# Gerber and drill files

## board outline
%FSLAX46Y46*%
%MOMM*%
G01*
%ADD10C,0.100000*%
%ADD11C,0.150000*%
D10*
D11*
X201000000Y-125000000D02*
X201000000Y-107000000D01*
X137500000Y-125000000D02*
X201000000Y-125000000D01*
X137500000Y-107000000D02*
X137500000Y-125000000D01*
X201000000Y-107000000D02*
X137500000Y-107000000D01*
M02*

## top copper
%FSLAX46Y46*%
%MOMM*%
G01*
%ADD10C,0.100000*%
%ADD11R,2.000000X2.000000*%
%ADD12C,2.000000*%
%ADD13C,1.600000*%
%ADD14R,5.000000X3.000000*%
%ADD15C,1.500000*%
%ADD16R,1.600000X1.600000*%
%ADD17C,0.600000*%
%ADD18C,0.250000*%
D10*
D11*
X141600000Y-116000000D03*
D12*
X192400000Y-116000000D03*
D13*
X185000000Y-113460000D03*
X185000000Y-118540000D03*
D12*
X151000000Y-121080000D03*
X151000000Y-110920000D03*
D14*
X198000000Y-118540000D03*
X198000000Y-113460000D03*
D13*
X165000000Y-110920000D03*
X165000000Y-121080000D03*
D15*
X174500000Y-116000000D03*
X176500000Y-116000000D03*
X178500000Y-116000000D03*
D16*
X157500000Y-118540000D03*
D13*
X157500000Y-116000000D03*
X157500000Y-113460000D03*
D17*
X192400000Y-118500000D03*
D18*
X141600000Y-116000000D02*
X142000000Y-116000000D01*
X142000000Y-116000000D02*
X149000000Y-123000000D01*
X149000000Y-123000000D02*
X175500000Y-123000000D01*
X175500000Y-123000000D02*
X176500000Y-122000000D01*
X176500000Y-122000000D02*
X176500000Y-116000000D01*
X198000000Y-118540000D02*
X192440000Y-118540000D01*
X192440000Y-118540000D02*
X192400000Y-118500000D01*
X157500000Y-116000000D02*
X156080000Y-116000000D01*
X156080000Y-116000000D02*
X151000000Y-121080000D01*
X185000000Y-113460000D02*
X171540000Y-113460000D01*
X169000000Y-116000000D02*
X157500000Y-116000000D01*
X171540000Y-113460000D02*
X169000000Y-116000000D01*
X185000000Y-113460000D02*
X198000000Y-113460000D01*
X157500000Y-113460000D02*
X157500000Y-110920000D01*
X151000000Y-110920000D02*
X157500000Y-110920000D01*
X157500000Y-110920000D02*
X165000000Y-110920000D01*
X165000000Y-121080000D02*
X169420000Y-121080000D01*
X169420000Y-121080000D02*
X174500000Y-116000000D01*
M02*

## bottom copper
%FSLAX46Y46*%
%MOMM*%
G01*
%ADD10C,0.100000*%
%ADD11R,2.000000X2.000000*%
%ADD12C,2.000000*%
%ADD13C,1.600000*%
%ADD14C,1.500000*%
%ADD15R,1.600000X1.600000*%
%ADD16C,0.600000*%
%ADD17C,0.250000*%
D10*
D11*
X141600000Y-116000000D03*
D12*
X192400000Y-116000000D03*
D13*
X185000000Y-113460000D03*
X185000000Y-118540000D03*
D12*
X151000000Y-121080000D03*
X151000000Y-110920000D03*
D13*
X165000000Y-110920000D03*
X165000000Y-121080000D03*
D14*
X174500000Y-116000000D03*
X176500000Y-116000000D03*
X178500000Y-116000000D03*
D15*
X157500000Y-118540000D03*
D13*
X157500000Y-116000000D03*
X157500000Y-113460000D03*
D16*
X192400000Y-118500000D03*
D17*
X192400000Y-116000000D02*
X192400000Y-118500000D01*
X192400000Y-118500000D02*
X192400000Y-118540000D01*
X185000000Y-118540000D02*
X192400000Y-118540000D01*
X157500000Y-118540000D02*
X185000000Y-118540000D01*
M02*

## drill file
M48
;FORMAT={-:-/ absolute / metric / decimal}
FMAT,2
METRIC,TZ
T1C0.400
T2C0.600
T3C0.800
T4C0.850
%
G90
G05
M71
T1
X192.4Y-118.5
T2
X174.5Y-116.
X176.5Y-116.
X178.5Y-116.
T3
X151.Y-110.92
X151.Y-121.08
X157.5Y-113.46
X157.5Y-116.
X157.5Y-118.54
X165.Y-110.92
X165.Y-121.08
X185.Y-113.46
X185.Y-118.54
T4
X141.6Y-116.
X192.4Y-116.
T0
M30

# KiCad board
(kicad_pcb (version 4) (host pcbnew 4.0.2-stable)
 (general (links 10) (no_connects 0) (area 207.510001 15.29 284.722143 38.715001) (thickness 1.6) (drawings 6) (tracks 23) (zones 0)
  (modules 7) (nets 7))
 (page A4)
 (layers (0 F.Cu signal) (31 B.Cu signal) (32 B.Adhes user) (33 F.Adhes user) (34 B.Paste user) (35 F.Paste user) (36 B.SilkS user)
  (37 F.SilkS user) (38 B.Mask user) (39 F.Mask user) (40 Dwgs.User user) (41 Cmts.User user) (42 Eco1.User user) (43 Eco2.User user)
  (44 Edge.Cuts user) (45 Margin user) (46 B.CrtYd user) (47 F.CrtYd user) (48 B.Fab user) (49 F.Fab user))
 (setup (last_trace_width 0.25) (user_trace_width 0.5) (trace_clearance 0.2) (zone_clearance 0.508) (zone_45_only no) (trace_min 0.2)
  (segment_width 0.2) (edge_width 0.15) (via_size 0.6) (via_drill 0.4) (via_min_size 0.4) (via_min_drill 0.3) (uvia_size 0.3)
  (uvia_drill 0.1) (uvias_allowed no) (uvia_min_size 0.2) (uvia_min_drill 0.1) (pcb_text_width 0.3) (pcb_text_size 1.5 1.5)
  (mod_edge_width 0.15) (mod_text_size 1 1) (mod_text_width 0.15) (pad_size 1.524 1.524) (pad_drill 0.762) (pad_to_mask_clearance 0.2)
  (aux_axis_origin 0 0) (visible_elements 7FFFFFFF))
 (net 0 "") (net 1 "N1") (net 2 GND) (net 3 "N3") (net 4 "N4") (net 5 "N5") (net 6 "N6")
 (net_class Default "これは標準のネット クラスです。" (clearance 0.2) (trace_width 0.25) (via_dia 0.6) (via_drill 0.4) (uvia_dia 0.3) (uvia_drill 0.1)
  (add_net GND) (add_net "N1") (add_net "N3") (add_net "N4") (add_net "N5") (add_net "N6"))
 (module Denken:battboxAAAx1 (layer B.Cu) (at 247.01 29.64)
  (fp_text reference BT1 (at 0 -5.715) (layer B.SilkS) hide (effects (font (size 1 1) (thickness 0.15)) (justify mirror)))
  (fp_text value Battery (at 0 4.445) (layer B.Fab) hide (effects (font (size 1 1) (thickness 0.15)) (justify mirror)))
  (pad 1 thru_hole rect (at -25.4 0) (size 2 2) (drill 0.85) (layers *.Cu *.Mask B.SilkS) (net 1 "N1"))
  (pad 2 thru_hole circle (at 25.4 0) (size 2 2) (drill 0.85) (layers *.Cu *.Mask B.SilkS) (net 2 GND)))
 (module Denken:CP (layer F.Cu) (at 265.01 29.64 270)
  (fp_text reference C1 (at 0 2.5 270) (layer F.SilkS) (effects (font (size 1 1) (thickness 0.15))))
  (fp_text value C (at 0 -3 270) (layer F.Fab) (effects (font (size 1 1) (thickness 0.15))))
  (pad 1 thru_hole circle (at -2.54 0 270) (size 1.6 1.6) (drill 0.8) (layers *.Cu *.Mask F.SilkS) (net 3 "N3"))
  (pad 2 thru_hole circle (at 2.54 0 270) (size 1.6 1.6) (drill 0.8) (layers *.Cu *.Mask F.SilkS) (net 2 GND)))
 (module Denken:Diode (layer F.Cu) (at 231.01 29.64 90)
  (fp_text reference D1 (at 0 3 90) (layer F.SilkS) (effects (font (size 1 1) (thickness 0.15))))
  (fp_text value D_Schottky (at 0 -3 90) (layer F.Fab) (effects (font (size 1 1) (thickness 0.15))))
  (pad 1 thru_hole circle (at -5.08 0 90) (size 2 2) (drill 0.8) (layers *.Cu *.Mask F.SilkS) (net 3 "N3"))
  (pad 2 thru_hole circle (at 5.08 0 90) (size 2 2) (drill 0.8) (layers *.Cu *.Mask F.SilkS) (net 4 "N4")))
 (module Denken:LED (layer F.Cu) (at 278.01 29.64 180)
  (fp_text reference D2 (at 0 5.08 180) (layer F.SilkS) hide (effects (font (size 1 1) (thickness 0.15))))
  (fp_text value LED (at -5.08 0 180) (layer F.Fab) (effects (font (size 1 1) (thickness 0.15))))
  (pad 1 smd rect (at 0 -2.54 180) (size 5 3) (layers F.Cu F.Paste F.Mask) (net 2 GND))
  (pad 2 smd rect (at 0 2.54 180) (size 5 3) (layers F.Cu F.Paste F.Mask) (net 3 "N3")))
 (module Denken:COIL (layer F.Cu) (at 245.01 29.64 270)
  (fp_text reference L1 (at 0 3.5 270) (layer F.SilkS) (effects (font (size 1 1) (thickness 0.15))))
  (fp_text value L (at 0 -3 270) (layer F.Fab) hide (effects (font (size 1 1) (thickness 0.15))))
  (pad 1 thru_hole circle (at -5.08 0 270) (size 1.6 1.6) (drill 0.8) (layers *.Cu *.Mask F.SilkS) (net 4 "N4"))
  (pad 2 thru_hole circle (at 5.08 0 270) (size 1.6 1.6) (drill 0.8) (layers *.Cu *.Mask F.SilkS) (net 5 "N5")))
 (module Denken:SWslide (layer F.Cu) (at 256.51 29.64)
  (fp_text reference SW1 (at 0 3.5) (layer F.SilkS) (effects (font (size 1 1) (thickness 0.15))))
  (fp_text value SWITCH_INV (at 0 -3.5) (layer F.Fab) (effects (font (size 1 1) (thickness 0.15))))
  (pad 1 thru_hole circle (at -2 0) (size 1.5 1.5) (drill 0.6) (layers *.Cu *.Mask F.SilkS) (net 5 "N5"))
  (pad 2 thru_hole circle (at 0 0) (size 1.5 1.5) (drill 0.6) (layers *.Cu *.Mask F.SilkS) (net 1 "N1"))
  (pad 3 thru_hole circle (at 2 0) (size 1.5 1.5) (drill 0.6) (layers *.Cu *.Mask F.SilkS) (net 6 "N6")))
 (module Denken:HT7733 (layer F.Cu) (at 237.51 29.64 90)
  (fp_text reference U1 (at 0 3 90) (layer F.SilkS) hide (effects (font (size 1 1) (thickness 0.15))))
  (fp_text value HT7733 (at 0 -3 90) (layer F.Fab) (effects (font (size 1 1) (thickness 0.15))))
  (pad 1 thru_hole rect (at -2.54 0 90) (size 1.6 1.6) (drill 0.8) (layers *.Cu *.Mask F.SilkS) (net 2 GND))
  (pad 2 thru_hole circle (at 0 0 90) (size 1.6 1.6) (drill 0.8) (layers *.Cu *.Mask F.SilkS) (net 3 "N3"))
  (pad 3 thru_hole circle (at 2.54 0 90) (size 1.6 1.6) (drill 0.8) (layers *.Cu *.Mask F.SilkS) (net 4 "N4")))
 (gr_line (start 281.01 38.64) (end 281.01 20.64) (angle 90) (layer Edge.Cuts) (width 0.15))
 (gr_line (start 217.51 38.64) (end 281.01 38.64) (angle 90) (layer Edge.Cuts) (width 0.15))
 (gr_line (start 217.51 20.64) (end 217.51 38.64) (angle 90) (layer Edge.Cuts) (width 0.15))
 (gr_line (start 281.01 20.64) (end 217.51 20.64) (angle 90) (layer Edge.Cuts) (width 0.15))
 (segment (start 221.61 29.64) (end 222.01 29.64) (width 0.25) (layer F.Cu) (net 1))
 (segment (start 222.01 29.64) (end 229.01 36.64) (width 0.25) (layer F.Cu) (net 1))
 (segment (start 229.01 36.64) (end 255.51 36.64) (width 0.25) (layer F.Cu) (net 1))
 (segment (start 255.51 36.64) (end 256.51 35.64) (width 0.25) (layer F.Cu) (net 1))
 (segment (start 256.51 35.64) (end 256.51 29.64) (width 0.25) (layer F.Cu) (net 1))
 (via (at 272.41 32.14) (size 0.6) (drill 0.4) (layers F.Cu B.Cu) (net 2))
 (segment (start 278.01 32.18) (end 272.45 32.18) (width 0.25) (layer F.Cu) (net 2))
 (segment (start 272.45 32.18) (end 272.41 32.14) (width 0.25) (layer F.Cu) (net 2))
 (segment (start 272.41 29.64) (end 272.41 32.14) (width 0.25) (layer B.Cu) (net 2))
 (segment (start 272.41 32.14) (end 272.41 32.18) (width 0.25) (layer B.Cu) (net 2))
 (segment (start 265.01 32.18) (end 272.41 32.18) (width 0.25) (layer B.Cu) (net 2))
 (segment (start 237.51 32.18) (end 265.01 32.18) (width 0.25) (layer B.Cu) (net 2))
 (segment (start 237.51 29.64) (end 236.09 29.64) (width 0.25) (layer F.Cu) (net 3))
 (segment (start 236.09 29.64) (end 231.01 34.72) (width 0.25) (layer F.Cu) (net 3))
 (segment (start 265.01 27.1) (end 251.55 27.1) (width 0.25) (layer F.Cu) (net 3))
 (segment (start 249.01 29.64) (end 237.51 29.64) (width 0.25) (layer F.Cu) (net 3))
 (segment (start 251.55 27.1) (end 249.01 29.64) (width 0.25) (layer F.Cu) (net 3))
 (segment (start 265.01 27.1) (end 278.01 27.1) (width 0.25) (layer F.Cu) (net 3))
 (segment (start 237.51 27.1) (end 237.51 24.56) (width 0.25) (layer F.Cu) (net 4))
 (segment (start 231.01 24.56) (end 237.51 24.56) (width 0.25) (layer F.Cu) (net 4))
 (segment (start 237.51 24.56) (end 245.01 24.56) (width 0.25) (layer F.Cu) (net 4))
 (segment (start 245.01 34.72) (end 249.43 34.72) (width 0.25) (layer F.Cu) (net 5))
 (segment (start 249.43 34.72) (end 254.51 29.64) (width 0.25) (layer F.Cu) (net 5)))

